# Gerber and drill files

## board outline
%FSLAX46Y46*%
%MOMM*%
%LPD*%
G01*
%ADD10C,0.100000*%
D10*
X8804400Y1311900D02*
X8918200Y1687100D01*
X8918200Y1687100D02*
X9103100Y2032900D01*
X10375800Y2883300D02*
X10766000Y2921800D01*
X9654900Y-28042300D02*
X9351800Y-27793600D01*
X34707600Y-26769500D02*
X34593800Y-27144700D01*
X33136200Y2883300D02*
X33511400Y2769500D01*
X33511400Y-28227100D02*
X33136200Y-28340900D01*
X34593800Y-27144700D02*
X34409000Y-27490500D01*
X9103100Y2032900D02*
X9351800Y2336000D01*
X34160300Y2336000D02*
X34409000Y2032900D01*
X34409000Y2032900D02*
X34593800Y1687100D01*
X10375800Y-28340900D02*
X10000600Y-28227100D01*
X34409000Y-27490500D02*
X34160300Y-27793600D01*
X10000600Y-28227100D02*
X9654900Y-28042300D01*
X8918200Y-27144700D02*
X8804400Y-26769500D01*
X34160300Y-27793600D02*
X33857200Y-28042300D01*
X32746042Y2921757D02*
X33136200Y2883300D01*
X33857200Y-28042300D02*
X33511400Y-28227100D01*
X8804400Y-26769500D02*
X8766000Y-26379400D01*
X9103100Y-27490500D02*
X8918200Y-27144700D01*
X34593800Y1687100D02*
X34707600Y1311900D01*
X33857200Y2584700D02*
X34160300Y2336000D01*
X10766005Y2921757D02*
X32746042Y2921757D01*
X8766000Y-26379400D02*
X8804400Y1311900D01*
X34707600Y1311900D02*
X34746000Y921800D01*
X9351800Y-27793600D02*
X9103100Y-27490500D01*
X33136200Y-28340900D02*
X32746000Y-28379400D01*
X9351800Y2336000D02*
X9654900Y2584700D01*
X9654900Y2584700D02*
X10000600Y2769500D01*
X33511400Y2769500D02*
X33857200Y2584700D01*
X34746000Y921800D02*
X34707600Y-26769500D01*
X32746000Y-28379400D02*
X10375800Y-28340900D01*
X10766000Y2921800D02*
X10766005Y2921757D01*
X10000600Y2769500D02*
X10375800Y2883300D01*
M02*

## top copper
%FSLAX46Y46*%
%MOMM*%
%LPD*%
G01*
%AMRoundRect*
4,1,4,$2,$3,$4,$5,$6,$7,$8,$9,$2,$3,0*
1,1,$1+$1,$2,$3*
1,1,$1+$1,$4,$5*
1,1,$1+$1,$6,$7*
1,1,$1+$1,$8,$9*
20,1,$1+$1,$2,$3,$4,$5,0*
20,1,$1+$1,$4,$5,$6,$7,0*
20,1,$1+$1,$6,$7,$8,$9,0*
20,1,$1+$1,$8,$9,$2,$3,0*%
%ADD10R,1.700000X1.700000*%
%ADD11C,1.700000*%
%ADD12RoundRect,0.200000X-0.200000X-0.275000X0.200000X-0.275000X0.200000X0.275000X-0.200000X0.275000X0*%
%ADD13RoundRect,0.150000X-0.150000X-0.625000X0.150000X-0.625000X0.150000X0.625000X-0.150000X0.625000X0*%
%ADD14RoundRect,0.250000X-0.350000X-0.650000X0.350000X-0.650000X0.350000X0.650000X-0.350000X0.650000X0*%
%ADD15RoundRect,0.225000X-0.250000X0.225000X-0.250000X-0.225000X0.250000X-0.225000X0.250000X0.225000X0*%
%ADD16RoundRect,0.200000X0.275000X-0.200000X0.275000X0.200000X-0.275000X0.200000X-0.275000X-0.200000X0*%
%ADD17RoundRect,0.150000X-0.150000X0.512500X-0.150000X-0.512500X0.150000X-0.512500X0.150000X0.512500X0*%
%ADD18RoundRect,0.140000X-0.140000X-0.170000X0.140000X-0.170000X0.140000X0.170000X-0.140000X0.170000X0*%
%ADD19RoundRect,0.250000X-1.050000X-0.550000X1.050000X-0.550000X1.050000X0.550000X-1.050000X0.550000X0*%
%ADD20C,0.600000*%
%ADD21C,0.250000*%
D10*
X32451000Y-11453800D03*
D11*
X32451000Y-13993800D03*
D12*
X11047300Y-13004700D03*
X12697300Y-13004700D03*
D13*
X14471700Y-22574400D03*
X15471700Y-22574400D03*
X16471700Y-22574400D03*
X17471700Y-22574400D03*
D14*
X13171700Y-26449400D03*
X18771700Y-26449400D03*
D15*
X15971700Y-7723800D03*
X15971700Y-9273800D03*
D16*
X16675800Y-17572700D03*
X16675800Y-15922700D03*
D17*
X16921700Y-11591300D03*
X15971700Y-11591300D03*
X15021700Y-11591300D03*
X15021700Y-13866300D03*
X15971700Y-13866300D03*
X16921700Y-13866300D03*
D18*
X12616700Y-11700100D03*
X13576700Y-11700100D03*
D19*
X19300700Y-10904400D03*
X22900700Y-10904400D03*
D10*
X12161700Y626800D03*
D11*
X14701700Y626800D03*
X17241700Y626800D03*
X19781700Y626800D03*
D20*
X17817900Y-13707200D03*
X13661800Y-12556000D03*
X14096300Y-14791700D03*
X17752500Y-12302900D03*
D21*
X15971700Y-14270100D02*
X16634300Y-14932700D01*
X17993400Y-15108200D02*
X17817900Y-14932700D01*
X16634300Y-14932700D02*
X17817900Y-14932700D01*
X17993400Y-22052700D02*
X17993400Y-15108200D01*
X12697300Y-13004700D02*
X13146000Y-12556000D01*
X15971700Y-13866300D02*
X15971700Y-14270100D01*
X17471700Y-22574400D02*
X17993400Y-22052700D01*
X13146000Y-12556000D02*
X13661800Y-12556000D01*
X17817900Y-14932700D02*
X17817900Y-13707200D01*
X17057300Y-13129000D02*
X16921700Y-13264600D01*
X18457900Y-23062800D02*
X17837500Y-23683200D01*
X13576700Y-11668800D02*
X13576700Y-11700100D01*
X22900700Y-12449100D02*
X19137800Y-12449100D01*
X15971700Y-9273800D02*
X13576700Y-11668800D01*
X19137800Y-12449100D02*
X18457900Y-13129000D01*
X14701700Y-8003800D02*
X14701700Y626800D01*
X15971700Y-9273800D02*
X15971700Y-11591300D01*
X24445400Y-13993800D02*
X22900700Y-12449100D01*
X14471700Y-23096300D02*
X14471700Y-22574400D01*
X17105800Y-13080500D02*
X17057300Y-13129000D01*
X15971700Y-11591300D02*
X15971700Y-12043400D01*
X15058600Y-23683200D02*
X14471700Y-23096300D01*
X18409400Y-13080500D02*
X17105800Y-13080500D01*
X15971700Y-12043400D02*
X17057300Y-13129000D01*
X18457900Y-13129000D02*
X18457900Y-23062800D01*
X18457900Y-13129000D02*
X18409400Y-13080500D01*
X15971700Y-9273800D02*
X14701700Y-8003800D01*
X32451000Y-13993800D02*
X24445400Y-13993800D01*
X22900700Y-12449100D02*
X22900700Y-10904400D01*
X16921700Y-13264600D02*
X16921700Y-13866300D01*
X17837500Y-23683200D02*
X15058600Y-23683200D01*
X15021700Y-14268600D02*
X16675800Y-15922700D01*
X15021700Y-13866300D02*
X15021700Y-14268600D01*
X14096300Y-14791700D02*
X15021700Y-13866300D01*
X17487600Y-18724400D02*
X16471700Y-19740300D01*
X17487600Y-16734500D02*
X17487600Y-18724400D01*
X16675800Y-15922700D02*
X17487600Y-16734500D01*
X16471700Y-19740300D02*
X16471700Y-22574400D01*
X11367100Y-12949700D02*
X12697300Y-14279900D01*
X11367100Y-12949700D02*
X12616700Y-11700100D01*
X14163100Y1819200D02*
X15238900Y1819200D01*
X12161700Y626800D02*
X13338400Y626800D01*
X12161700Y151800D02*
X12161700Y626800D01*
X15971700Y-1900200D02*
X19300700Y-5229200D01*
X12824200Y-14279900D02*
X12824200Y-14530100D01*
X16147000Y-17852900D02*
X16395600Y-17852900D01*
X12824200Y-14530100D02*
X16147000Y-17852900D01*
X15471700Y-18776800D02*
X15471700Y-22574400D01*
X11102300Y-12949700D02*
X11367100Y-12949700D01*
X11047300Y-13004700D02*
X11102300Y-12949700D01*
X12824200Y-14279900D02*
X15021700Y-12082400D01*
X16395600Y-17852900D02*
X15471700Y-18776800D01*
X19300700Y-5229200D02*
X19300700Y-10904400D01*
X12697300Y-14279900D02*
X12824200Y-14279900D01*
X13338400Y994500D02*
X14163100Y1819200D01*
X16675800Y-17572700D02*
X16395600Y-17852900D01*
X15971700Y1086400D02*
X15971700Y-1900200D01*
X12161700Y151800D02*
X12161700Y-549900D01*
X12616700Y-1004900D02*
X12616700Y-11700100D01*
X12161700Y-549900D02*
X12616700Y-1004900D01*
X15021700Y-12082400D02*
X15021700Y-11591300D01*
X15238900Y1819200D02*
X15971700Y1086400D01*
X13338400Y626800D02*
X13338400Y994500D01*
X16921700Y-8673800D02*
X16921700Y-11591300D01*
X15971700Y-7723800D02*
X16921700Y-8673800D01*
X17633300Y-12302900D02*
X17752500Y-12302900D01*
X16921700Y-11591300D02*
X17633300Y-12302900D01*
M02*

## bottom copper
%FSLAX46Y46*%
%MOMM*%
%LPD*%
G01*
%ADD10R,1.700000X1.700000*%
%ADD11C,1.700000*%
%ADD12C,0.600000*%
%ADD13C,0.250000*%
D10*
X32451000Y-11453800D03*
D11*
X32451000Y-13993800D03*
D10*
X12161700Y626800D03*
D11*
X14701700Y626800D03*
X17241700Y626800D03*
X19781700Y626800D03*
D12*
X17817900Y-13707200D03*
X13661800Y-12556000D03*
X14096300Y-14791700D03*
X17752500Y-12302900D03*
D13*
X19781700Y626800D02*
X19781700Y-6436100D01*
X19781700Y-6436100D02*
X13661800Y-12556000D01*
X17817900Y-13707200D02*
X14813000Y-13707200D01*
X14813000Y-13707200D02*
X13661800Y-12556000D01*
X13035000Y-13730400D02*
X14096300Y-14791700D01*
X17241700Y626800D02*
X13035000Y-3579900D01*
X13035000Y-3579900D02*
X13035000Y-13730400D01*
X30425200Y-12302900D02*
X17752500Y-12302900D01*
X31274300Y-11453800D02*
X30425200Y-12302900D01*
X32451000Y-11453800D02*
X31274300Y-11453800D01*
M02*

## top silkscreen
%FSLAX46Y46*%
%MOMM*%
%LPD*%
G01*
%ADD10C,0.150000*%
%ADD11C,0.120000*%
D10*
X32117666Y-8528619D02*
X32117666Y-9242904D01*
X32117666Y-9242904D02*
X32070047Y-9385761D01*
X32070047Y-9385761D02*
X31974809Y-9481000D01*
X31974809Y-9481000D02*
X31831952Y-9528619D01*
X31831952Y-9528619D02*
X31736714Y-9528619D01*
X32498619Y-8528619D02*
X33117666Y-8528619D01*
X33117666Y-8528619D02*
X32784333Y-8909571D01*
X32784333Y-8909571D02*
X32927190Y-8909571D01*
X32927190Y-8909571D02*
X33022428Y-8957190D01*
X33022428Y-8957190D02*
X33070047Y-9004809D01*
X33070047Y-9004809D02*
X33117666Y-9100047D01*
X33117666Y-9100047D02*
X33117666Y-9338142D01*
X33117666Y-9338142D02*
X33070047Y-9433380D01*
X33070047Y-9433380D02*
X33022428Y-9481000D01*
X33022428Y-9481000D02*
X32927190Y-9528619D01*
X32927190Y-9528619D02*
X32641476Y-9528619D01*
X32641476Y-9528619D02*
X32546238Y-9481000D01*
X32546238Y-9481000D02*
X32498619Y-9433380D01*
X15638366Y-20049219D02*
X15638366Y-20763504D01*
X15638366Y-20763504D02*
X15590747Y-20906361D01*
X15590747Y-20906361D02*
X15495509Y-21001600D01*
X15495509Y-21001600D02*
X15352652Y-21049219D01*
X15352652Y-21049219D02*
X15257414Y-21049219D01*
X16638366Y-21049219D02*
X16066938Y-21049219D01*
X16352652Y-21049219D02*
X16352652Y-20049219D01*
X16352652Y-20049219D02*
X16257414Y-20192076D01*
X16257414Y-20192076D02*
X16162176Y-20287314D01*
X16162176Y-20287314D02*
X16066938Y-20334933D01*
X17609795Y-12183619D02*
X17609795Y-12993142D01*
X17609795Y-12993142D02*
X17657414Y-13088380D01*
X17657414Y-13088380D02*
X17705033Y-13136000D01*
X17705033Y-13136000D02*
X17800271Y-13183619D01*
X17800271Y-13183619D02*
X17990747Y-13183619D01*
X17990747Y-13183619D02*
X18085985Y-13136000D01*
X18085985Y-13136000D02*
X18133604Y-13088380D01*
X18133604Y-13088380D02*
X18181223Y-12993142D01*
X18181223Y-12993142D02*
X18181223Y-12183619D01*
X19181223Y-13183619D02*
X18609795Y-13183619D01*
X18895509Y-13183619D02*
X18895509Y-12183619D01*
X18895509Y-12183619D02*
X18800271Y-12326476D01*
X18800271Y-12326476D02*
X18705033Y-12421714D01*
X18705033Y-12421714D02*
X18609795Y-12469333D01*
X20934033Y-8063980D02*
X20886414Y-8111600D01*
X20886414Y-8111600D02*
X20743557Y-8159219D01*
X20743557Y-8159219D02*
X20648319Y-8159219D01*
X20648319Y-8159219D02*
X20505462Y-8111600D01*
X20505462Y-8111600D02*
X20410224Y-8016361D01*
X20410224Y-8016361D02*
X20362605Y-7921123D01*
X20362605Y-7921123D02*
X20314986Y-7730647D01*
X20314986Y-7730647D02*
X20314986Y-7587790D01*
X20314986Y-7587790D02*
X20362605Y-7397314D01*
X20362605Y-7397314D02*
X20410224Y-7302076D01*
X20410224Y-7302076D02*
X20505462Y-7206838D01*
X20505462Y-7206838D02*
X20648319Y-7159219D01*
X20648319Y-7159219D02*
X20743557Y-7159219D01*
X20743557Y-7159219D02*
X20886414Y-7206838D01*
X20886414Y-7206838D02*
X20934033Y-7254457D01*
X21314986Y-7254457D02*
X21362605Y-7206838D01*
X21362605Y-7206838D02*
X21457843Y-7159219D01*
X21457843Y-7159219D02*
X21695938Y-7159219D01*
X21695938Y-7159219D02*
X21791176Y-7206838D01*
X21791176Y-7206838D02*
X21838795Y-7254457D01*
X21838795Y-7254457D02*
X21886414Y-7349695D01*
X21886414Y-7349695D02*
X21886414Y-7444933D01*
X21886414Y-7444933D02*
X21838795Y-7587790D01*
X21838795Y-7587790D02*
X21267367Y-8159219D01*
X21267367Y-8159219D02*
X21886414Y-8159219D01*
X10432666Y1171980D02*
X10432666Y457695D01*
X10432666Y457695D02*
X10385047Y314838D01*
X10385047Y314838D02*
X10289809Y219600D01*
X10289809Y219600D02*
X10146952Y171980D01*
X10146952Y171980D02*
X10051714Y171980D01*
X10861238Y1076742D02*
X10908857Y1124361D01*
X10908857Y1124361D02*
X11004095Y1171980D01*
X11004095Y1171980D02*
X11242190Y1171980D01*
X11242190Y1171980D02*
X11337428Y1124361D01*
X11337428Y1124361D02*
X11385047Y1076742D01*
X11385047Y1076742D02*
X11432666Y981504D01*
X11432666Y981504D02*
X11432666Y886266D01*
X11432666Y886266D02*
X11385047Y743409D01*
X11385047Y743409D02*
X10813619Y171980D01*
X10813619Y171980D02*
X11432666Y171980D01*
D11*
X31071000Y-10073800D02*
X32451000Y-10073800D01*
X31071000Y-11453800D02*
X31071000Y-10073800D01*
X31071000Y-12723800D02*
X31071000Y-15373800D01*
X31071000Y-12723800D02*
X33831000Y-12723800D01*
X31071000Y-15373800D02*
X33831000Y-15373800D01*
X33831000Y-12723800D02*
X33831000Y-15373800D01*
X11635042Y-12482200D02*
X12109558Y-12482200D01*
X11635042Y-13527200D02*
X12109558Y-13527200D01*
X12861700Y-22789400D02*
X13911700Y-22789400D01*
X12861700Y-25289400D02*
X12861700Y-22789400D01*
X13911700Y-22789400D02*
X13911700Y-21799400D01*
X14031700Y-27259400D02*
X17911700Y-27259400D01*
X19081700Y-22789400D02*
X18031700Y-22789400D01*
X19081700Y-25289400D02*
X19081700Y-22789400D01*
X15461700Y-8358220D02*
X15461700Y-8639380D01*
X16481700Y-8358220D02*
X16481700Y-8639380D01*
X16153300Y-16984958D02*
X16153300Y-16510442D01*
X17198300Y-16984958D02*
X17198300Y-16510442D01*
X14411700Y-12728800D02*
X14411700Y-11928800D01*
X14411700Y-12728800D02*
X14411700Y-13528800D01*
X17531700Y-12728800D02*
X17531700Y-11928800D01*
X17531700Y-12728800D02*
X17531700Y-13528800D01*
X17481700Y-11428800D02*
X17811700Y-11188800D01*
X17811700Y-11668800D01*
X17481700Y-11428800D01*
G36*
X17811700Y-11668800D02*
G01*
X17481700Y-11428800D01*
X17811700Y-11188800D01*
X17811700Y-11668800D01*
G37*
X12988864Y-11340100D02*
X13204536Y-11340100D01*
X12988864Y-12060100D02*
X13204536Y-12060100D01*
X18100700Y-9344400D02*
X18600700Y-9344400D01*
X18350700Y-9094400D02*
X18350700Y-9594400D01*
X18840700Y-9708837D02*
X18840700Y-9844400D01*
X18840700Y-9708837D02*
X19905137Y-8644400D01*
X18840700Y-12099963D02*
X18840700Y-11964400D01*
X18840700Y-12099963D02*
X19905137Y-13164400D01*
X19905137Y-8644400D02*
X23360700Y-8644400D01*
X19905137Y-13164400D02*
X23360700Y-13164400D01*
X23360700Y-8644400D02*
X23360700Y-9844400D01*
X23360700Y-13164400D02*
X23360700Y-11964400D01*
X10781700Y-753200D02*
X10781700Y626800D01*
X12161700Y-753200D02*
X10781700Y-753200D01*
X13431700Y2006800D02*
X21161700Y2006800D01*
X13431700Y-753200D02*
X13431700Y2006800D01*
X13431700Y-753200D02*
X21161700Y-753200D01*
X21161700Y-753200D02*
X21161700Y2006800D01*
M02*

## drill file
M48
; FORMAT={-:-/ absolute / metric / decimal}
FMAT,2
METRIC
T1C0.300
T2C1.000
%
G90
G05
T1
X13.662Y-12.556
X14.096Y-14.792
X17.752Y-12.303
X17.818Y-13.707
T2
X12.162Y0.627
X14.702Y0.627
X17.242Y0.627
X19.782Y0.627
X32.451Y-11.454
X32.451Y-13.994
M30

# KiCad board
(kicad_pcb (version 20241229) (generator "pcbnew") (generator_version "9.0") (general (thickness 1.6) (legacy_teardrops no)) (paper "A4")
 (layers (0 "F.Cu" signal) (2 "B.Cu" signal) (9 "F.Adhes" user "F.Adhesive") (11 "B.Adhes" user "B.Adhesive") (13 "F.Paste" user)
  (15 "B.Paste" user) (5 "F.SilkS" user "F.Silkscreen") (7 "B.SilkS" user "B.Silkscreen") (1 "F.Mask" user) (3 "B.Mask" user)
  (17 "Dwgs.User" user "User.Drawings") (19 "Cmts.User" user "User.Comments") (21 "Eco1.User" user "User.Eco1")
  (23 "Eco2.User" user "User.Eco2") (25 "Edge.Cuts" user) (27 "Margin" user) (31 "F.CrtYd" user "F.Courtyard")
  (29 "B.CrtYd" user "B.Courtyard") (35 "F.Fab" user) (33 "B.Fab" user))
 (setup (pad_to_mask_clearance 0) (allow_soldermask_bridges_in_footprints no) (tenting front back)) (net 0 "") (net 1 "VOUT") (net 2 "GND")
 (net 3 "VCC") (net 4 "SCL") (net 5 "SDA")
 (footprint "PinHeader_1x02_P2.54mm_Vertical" (layer "F.Cu") (at 32.451 11.4538)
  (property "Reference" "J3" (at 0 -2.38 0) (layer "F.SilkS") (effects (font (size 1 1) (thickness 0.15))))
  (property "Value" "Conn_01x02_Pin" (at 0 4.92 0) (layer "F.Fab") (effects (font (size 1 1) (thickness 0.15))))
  (fp_line (start -1.38 -1.38) (end 0 -1.38) (stroke (width 0.12) (type solid)) (layer "F.SilkS"))
  (fp_line (start -1.38 0) (end -1.38 -1.38) (stroke (width 0.12) (type solid)) (layer "F.SilkS"))
  (fp_line (start -1.38 1.27) (end -1.38 3.92) (stroke (width 0.12) (type solid)) (layer "F.SilkS"))
  (fp_line (start -1.38 1.27) (end 1.38 1.27) (stroke (width 0.12) (type solid)) (layer "F.SilkS"))
  (fp_line (start -1.38 3.92) (end 1.38 3.92) (stroke (width 0.12) (type solid)) (layer "F.SilkS"))
  (fp_line (start 1.38 1.27) (end 1.38 3.92) (stroke (width 0.12) (type solid)) (layer "F.SilkS"))
  (pad "1" thru_hole rect (at 0 0) (size 1.7 1.7) (drill 1) (layers "*.Cu" "*.Mask") (remove_unused_layers no) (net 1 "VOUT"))
  (pad "2" thru_hole circle (at 0 2.54) (size 1.7 1.7) (drill 1) (layers "*.Cu" "*.Mask") (remove_unused_layers no) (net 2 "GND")))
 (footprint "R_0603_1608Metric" (layer "F.Cu") (at 11.8723 13.0047)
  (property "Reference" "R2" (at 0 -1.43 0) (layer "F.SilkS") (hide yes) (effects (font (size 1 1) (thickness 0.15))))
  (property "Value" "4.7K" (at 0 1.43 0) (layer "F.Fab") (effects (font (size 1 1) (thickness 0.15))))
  (fp_line (start -0.237258 -0.5225) (end 0.237258 -0.5225) (stroke (width 0.12) (type solid)) (layer "F.SilkS"))
  (fp_line (start -0.237258 0.5225) (end 0.237258 0.5225) (stroke (width 0.12) (type solid)) (layer "F.SilkS"))
  (pad "1" smd roundrect (at -0.825 0) (size 0.8 0.95) (layers "F.Cu" "F.Mask" "F.Paste") (roundrect_rratio 0.25) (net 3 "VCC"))
  (pad "2" smd roundrect (at 0.825 0) (size 0.8 0.95) (layers "F.Cu" "F.Mask" "F.Paste") (roundrect_rratio 0.25) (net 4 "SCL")))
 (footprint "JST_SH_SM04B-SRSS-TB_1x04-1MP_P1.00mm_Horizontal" (layer "F.Cu") (at 15.9717 24.5744)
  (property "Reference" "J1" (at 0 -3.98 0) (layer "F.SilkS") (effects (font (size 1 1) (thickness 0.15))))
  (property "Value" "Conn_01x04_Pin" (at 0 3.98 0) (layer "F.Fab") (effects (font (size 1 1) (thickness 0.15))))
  (fp_line (start -3.11 -1.785) (end -2.06 -1.785) (stroke (width 0.12) (type solid)) (layer "F.SilkS"))
  (fp_line (start -3.11 0.715) (end -3.11 -1.785) (stroke (width 0.12) (type solid)) (layer "F.SilkS"))
  (fp_line (start -2.06 -1.785) (end -2.06 -2.775) (stroke (width 0.12) (type solid)) (layer "F.SilkS"))
  (fp_line (start -1.94 2.685) (end 1.94 2.685) (stroke (width 0.12) (type solid)) (layer "F.SilkS"))
  (fp_line (start 3.11 -1.785) (end 2.06 -1.785) (stroke (width 0.12) (type solid)) (layer "F.SilkS"))
  (fp_line (start 3.11 0.715) (end 3.11 -1.785) (stroke (width 0.12) (type solid)) (layer "F.SilkS"))
  (pad "1" smd roundrect (at -1.5 -2) (size 0.6 1.55) (layers "F.Cu" "F.Mask" "F.Paste") (roundrect_rratio 0.25) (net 2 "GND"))
  (pad "2" smd roundrect (at -0.5 -2) (size 0.6 1.55) (layers "F.Cu" "F.Mask" "F.Paste") (roundrect_rratio 0.25) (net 3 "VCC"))
  (pad "3" smd roundrect (at 0.5 -2) (size 0.6 1.55) (layers "F.Cu" "F.Mask" "F.Paste") (roundrect_rratio 0.25) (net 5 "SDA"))
  (pad "4" smd roundrect (at 1.5 -2) (size 0.6 1.55) (layers "F.Cu" "F.Mask" "F.Paste") (roundrect_rratio 0.25) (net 4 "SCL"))
  (pad "MP" smd roundrect (at -2.8 1.875) (size 1.2 1.8) (layers "F.Cu" "F.Mask" "F.Paste") (roundrect_rratio 0.208333))
  (pad "MP" smd roundrect (at 2.8 1.875) (size 1.2 1.8) (layers "F.Cu" "F.Mask" "F.Paste") (roundrect_rratio 0.208333)))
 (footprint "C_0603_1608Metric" (layer "F.Cu") (at 15.9717 8.4988 -90)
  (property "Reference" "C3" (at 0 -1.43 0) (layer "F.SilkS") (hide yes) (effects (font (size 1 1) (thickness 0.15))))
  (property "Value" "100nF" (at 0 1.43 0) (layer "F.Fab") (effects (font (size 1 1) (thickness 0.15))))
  (fp_line (start -0.14058 0.51) (end 0.14058 0.51) (stroke (width 0.12) (type solid)) (layer "F.SilkS"))
  (fp_line (start -0.14058 -0.51) (end 0.14058 -0.51) (stroke (width 0.12) (type solid)) (layer "F.SilkS"))
  (pad "1" smd roundrect (at -0.775 0 270) (size 0.9 0.95) (layers "F.Cu" "F.Mask" "F.Paste") (roundrect_rratio 0.25) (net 1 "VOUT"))
  (pad "2" smd roundrect (at 0.775 0 270) (size 0.9 0.95) (layers "F.Cu" "F.Mask" "F.Paste") (roundrect_rratio 0.25) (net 2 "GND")))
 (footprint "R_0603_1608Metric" (layer "F.Cu") (at 16.6758 16.7477 90)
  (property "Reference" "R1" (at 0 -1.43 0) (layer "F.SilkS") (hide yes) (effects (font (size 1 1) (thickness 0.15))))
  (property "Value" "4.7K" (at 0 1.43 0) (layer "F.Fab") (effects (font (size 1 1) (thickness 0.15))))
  (fp_line (start -0.237258 -0.5225) (end 0.237258 -0.5225) (stroke (width 0.12) (type solid)) (layer "F.SilkS"))
  (fp_line (start -0.237258 0.5225) (end 0.237258 0.5225) (stroke (width 0.12) (type solid)) (layer "F.SilkS"))
  (pad "1" smd roundrect (at -0.825 0 90) (size 0.8 0.95) (layers "F.Cu" "F.Mask" "F.Paste") (roundrect_rratio 0.25) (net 3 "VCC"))
  (pad "2" smd roundrect (at 0.825 0 90) (size 0.8 0.95) (layers "F.Cu" "F.Mask" "F.Paste") (roundrect_rratio 0.25) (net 5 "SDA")))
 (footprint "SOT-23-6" (layer "F.Cu") (at 15.9717 12.7288 -90)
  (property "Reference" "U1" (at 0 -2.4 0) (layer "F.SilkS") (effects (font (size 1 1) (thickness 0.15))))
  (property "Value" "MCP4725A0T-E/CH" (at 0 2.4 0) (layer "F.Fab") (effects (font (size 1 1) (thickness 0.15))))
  (fp_line (start 0 1.56) (end -0.8 1.56) (stroke (width 0.12) (type solid)) (layer "F.SilkS"))
  (fp_line (start 0 1.56) (end 0.8 1.56) (stroke (width 0.12) (type solid)) (layer "F.SilkS"))
  (fp_line (start 0 -1.56) (end -0.8 -1.56) (stroke (width 0.12) (type solid)) (layer "F.SilkS"))
  (fp_line (start 0 -1.56) (end 0.8 -1.56) (stroke (width 0.12) (type solid)) (layer "F.SilkS"))
  (fp_poly (pts (xy -1.3 -1.51) (xy -1.54 -1.84) (xy -1.06 -1.84)) (stroke (width 0.12) (type solid)) (fill yes) (layer "F.SilkS"))
  (pad "1" smd roundrect (at -1.1375 -0.95 270) (size 1.325 0.6) (layers "F.Cu" "F.Mask" "F.Paste") (roundrect_rratio 0.25) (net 1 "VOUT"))
  (pad "2" smd roundrect (at -1.1375 0 270) (size 1.325 0.6) (layers "F.Cu" "F.Mask" "F.Paste") (roundrect_rratio 0.25) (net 2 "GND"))
  (pad "3" smd roundrect (at -1.1375 0.95 270) (size 1.325 0.6) (layers "F.Cu" "F.Mask" "F.Paste") (roundrect_rratio 0.25) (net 3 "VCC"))
  (pad "4" smd roundrect (at 1.1375 0.95 270) (size 1.325 0.6) (layers "F.Cu" "F.Mask" "F.Paste") (roundrect_rratio 0.25) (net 5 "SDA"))
  (pad "5" smd roundrect (at 1.1375 0 270) (size 1.325 0.6) (layers "F.Cu" "F.Mask" "F.Paste") (roundrect_rratio 0.25) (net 4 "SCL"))
  (pad "6" smd roundrect (at 1.1375 -0.95 270) (size 1.325 0.6) (layers "F.Cu" "F.Mask" "F.Paste") (roundrect_rratio 0.25) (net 2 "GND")))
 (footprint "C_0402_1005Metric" (layer "F.Cu") (at 13.0967 11.7001)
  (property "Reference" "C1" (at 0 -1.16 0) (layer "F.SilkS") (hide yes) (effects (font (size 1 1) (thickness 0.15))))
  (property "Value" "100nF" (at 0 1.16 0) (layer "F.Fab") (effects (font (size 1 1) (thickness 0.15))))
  (fp_line (start -0.107836 -0.36) (end 0.107836 -0.36) (stroke (width 0.12) (type solid)) (layer "F.SilkS"))
  (fp_line (start -0.107836 0.36) (end 0.107836 0.36) (stroke (width 0.12) (type solid)) (layer "F.SilkS"))
  (pad "1" smd roundrect (at -0.48 0) (size 0.56 0.62) (layers "F.Cu" "F.Mask" "F.Paste") (roundrect_rratio 0.25) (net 3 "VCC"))
  (pad "2" smd roundrect (at 0.48 0) (size 0.56 0.62) (layers "F.Cu" "F.Mask" "F.Paste") (roundrect_rratio 0.25) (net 2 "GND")))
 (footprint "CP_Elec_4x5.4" (layer "F.Cu") (at 21.1007 10.9044)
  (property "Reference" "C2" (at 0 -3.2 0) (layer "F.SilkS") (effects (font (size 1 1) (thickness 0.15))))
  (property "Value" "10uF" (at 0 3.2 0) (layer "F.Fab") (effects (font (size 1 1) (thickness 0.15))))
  (fp_line (start -3 -1.56) (end -2.5 -1.56) (stroke (width 0.12) (type solid)) (layer "F.SilkS"))
  (fp_line (start -2.75 -1.81) (end -2.75 -1.31) (stroke (width 0.12) (type solid)) (layer "F.SilkS"))
  (fp_line (start -2.26 -1.195563) (end -2.26 -1.06) (stroke (width 0.12) (type solid)) (layer "F.SilkS"))
  (fp_line (start -2.26 -1.195563) (end -1.195563 -2.26) (stroke (width 0.12) (type solid)) (layer "F.SilkS"))
  (fp_line (start -2.26 1.195563) (end -2.26 1.06) (stroke (width 0.12) (type solid)) (layer "F.SilkS"))
  (fp_line (start -2.26 1.195563) (end -1.195563 2.26) (stroke (width 0.12) (type solid)) (layer "F.SilkS"))
  (fp_line (start -1.195563 -2.26) (end 2.26 -2.26) (stroke (width 0.12) (type solid)) (layer "F.SilkS"))
  (fp_line (start -1.195563 2.26) (end 2.26 2.26) (stroke (width 0.12) (type solid)) (layer "F.SilkS"))
  (fp_line (start 2.26 -2.26) (end 2.26 -1.06) (stroke (width 0.12) (type solid)) (layer "F.SilkS"))
  (fp_line (start 2.26 2.26) (end 2.26 1.06) (stroke (width 0.12) (type solid)) (layer "F.SilkS"))
  (pad "1" smd roundrect (at -1.8 0) (size 2.6 1.6) (layers "F.Cu" "F.Mask" "F.Paste") (roundrect_rratio 0.15625) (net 3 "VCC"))
  (pad "2" smd roundrect (at 1.8 0) (size 2.6 1.6) (layers "F.Cu" "F.Mask" "F.Paste") (roundrect_rratio 0.15625) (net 2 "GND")))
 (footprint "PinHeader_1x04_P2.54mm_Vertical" (layer "F.Cu") (at 12.1617 -0.6268 90)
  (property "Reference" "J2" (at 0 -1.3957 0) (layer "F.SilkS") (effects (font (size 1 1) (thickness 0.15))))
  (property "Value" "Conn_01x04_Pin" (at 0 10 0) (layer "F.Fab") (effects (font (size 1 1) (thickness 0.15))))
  (fp_line (start -1.38 -1.38) (end 0 -1.38) (stroke (width 0.12) (type solid)) (layer "F.SilkS"))
  (fp_line (start -1.38 0) (end -1.38 -1.38) (stroke (width 0.12) (type solid)) (layer "F.SilkS"))
  (fp_line (start 1.38 1.27) (end 1.38 9) (stroke (width 0.12) (type solid)) (layer "F.SilkS"))
  (fp_line (start -1.38 1.27) (end 1.38 1.27) (stroke (width 0.12) (type solid)) (layer "F.SilkS"))
  (fp_line (start -1.38 1.27) (end -1.38 9) (stroke (width 0.12) (type solid)) (layer "F.SilkS"))
  (fp_line (start -1.38 9) (end 1.38 9) (stroke (width 0.12) (type solid)) (layer "F.SilkS"))
  (pad "1" thru_hole rect (at 0 0 90) (size 1.7 1.7) (drill 1) (layers "*.Cu" "*.Mask") (remove_unused_layers no) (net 3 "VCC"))
  (pad "2" thru_hole circle (at 0 2.54 90) (size 1.7 1.7) (drill 1) (layers "*.Cu" "*.Mask") (remove_unused_layers no) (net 2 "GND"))
  (pad "3" thru_hole circle (at 0 5.08 90) (size 1.7 1.7) (drill 1) (layers "*.Cu" "*.Mask") (remove_unused_layers no) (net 5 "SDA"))
  (pad "4" thru_hole circle (at 0 7.62 90) (size 1.7 1.7) (drill 1) (layers "*.Cu" "*.Mask") (remove_unused_layers no) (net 4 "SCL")))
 (gr_line (start 8.8044 -1.3119) (end 8.9182 -1.6871) (stroke (width 0.1) (type solid)) (layer "Edge.Cuts"))
 (gr_line (start 8.9182 -1.6871) (end 9.1031 -2.0329) (stroke (width 0.1) (type solid)) (layer "Edge.Cuts"))
 (gr_line (start 10.3758 -2.8833) (end 10.766 -2.9218) (stroke (width 0.1) (type solid)) (layer "Edge.Cuts"))
 (gr_line (start 9.6549 28.0423) (end 9.3518 27.7936) (stroke (width 0.1) (type solid)) (layer "Edge.Cuts"))
 (gr_line (start 34.7076 26.7695) (end 34.5938 27.1447) (stroke (width 0.1) (type solid)) (layer "Edge.Cuts"))
 (gr_line (start 33.1362 -2.8833) (end 33.5114 -2.7695) (stroke (width 0.1) (type solid)) (layer "Edge.Cuts"))
 (gr_line (start 33.5114 28.2271) (end 33.1362 28.3409) (stroke (width 0.1) (type solid)) (layer "Edge.Cuts"))
 (gr_line (start 34.5938 27.1447) (end 34.409 27.4905) (stroke (width 0.1) (type solid)) (layer "Edge.Cuts"))
 (gr_line (start 9.1031 -2.0329) (end 9.3518 -2.336) (stroke (width 0.1) (type solid)) (layer "Edge.Cuts"))
 (gr_line (start 34.1603 -2.336) (end 34.409 -2.0329) (stroke (width 0.1) (type solid)) (layer "Edge.Cuts"))
 (gr_line (start 34.409 -2.0329) (end 34.5938 -1.6871) (stroke (width 0.1) (type solid)) (layer "Edge.Cuts"))
 (gr_line (start 10.3758 28.3409) (end 10.0006 28.2271) (stroke (width 0.1) (type solid)) (layer "Edge.Cuts"))
 (gr_line (start 34.409 27.4905) (end 34.1603 27.7936) (stroke (width 0.1) (type solid)) (layer "Edge.Cuts"))
 (gr_line (start 10.0006 28.2271) (end 9.6549 28.0423) (stroke (width 0.1) (type solid)) (layer "Edge.Cuts"))
 (gr_line (start 8.9182 27.1447) (end 8.8044 26.7695) (stroke (width 0.1) (type solid)) (layer "Edge.Cuts"))
 (gr_line (start 34.1603 27.7936) (end 33.8572 28.0423) (stroke (width 0.1) (type solid)) (layer "Edge.Cuts"))
 (gr_line (start 32.746042 -2.921757) (end 33.1362 -2.8833) (stroke (width 0.1) (type solid)) (layer "Edge.Cuts"))
 (gr_line (start 33.8572 28.0423) (end 33.5114 28.2271) (stroke (width 0.1) (type solid)) (layer "Edge.Cuts"))
 (gr_line (start 8.8044 26.7695) (end 8.766 26.3794) (stroke (width 0.1) (type solid)) (layer "Edge.Cuts"))
 (gr_line (start 9.1031 27.4905) (end 8.9182 27.1447) (stroke (width 0.1) (type solid)) (layer "Edge.Cuts"))
 (gr_line (start 34.5938 -1.6871) (end 34.7076 -1.3119) (stroke (width 0.1) (type solid)) (layer "Edge.Cuts"))
 (gr_line (start 33.8572 -2.5847) (end 34.1603 -2.336) (stroke (width 0.1) (type solid)) (layer "Edge.Cuts"))
 (gr_line (start 10.766005 -2.921757) (end 32.746042 -2.921757) (stroke (width 0.1) (type solid)) (layer "Edge.Cuts"))
 (gr_line (start 8.766 26.3794) (end 8.8044 -1.3119) (stroke (width 0.1) (type solid)) (layer "Edge.Cuts"))
 (gr_line (start 34.7076 -1.3119) (end 34.746 -0.9218) (stroke (width 0.1) (type solid)) (layer "Edge.Cuts"))
 (gr_line (start 9.3518 27.7936) (end 9.1031 27.4905) (stroke (width 0.1) (type solid)) (layer "Edge.Cuts"))
 (gr_line (start 33.1362 28.3409) (end 32.746 28.3794) (stroke (width 0.1) (type solid)) (layer "Edge.Cuts"))
 (gr_line (start 9.3518 -2.336) (end 9.6549 -2.5847) (stroke (width 0.1) (type solid)) (layer "Edge.Cuts"))
 (gr_line (start 9.6549 -2.5847) (end 10.0006 -2.7695) (stroke (width 0.1) (type solid)) (layer "Edge.Cuts"))
 (gr_line (start 33.5114 -2.7695) (end 33.8572 -2.5847) (stroke (width 0.1) (type solid)) (layer "Edge.Cuts"))
 (gr_line (start 34.746 -0.9218) (end 34.7076 26.7695) (stroke (width 0.1) (type solid)) (layer "Edge.Cuts"))
 (gr_line (start 32.746 28.3794) (end 10.3758 28.3409) (stroke (width 0.1) (type solid)) (layer "Edge.Cuts"))
 (gr_line (start 10.766 -2.9218) (end 10.766005 -2.921757) (stroke (width 0.1) (type solid)) (layer "Edge.Cuts"))
 (gr_line (start 10.0006 -2.7695) (end 10.3758 -2.8833) (stroke (width 0.1) (type solid)) (layer "Edge.Cuts"))
 (segment (start 15.9717 14.2701) (end 16.6343 14.9327) (width 0.25) (layer "F.Cu") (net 4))
 (segment (start 17.9934 15.1082) (end 17.8179 14.9327) (width 0.25) (layer "F.Cu") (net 4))
 (segment (start 16.6343 14.9327) (end 17.8179 14.9327) (width 0.25) (layer "F.Cu") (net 4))
 (segment (start 17.9934 22.0527) (end 17.9934 15.1082) (width 0.25) (layer "F.Cu") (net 4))
 (segment (start 12.6973 13.0047) (end 13.146 12.556) (width 0.25) (layer "F.Cu") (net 4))
 (segment (start 15.9717 13.8663) (end 15.9717 14.2701) (width 0.25) (layer "F.Cu") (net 4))
 (segment (start 17.4717 22.5744) (end 17.9934 22.0527) (width 0.25) (layer "F.Cu") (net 4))
 (segment (start 13.146 12.556) (end 13.6618 12.556) (width 0.25) (layer "F.Cu") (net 4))
 (segment (start 17.8179 14.9327) (end 17.8179 13.7072) (width 0.25) (layer "F.Cu") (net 4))
 (via (at 17.8179 13.7072) (size 0.6) (drill 0.3) (layers "F.Cu" "B.Cu") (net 4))
 (via (at 13.6618 12.556) (size 0.6) (drill 0.3) (layers "F.Cu" "B.Cu") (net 4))
 (segment (start 19.7817 -0.6268) (end 19.7817 6.4361) (width 0.25) (layer "B.Cu") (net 4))
 (segment (start 19.7817 6.4361) (end 13.6618 12.556) (width 0.25) (layer "B.Cu") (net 4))
 (segment (start 17.8179 13.7072) (end 14.813 13.7072) (width 0.25) (layer "B.Cu") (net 4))
 (segment (start 14.813 13.7072) (end 13.6618 12.556) (width 0.25) (layer "B.Cu") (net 4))
 (segment (start 17.0573 13.129) (end 16.9217 13.2646) (width 0.25) (layer "F.Cu") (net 2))
 (segment (start 18.4579 23.0628) (end 17.8375 23.6832) (width 0.25) (layer "F.Cu") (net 2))
 (segment (start 13.5767 11.6688) (end 13.5767 11.7001) (width 0.25) (layer "F.Cu") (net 2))
 (segment (start 22.9007 12.4491) (end 19.1378 12.4491) (width 0.25) (layer "F.Cu") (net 2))
 (segment (start 15.9717 9.2738) (end 13.5767 11.6688) (width 0.25) (layer "F.Cu") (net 2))
 (segment (start 19.1378 12.4491) (end 18.4579 13.129) (width 0.25) (layer "F.Cu") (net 2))
 (segment (start 14.7017 8.0038) (end 14.7017 -0.6268) (width 0.25) (layer "F.Cu") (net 2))
 (segment (start 15.9717 9.2738) (end 15.9717 11.5913) (width 0.25) (layer "F.Cu") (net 2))
 (segment (start 24.4454 13.9938) (end 22.9007 12.4491) (width 0.25) (layer "F.Cu") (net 2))
 (segment (start 14.4717 23.0963) (end 14.4717 22.5744) (width 0.25) (layer "F.Cu") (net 2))
 (segment (start 17.1058 13.0805) (end 17.0573 13.129) (width 0.25) (layer "F.Cu") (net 2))
 (segment (start 15.9717 11.5913) (end 15.9717 12.0434) (width 0.25) (layer "F.Cu") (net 2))
 (segment (start 15.0586 23.6832) (end 14.4717 23.0963) (width 0.25) (layer "F.Cu") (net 2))
 (segment (start 18.4094 13.0805) (end 17.1058 13.0805) (width 0.25) (layer "F.Cu") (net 2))
 (segment (start 15.9717 12.0434) (end 17.0573 13.129) (width 0.25) (layer "F.Cu") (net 2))
 (segment (start 18.4579 13.129) (end 18.4579 23.0628) (width 0.25) (layer "F.Cu") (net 2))
 (segment (start 18.4579 13.129) (end 18.4094 13.0805) (width 0.25) (layer "F.Cu") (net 2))
 (segment (start 15.9717 9.2738) (end 14.7017 8.0038) (width 0.25) (layer "F.Cu") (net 2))
 (segment (start 32.451 13.9938) (end 24.4454 13.9938) (width 0.25) (layer "F.Cu") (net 2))
 (segment (start 22.9007 12.4491) (end 22.9007 10.9044) (width 0.25) (layer "F.Cu") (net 2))
 (segment (start 16.9217 13.2646) (end 16.9217 13.8663) (width 0.25) (layer "F.Cu") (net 2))
 (segment (start 17.8375 23.6832) (end 15.0586 23.6832) (width 0.25) (layer "F.Cu") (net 2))
 (segment (start 15.0217 14.2686) (end 16.6758 15.9227) (width 0.25) (layer "F.Cu") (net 5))
 (segment (start 15.0217 13.8663) (end 15.0217 14.2686) (width 0.25) (layer "F.Cu") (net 5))
 (segment (start 14.0963 14.7917) (end 15.0217 13.8663) (width 0.25) (layer "F.Cu") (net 5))
 (segment (start 17.4876 18.7244) (end 16.4717 19.7403) (width 0.25) (layer "F.Cu") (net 5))
 (segment (start 17.4876 16.7345) (end 17.4876 18.7244) (width 0.25) (layer "F.Cu") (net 5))
 (segment (start 16.6758 15.9227) (end 17.4876 16.7345) (width 0.25) (layer "F.Cu") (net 5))
 (segment (start 16.4717 19.7403) (end 16.4717 22.5744) (width 0.25) (layer "F.Cu") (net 5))
 (via (at 14.0963 14.7917) (size 0.6) (drill 0.3) (layers "F.Cu" "B.Cu") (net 5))
 (segment (start 13.035 13.7304) (end 14.0963 14.7917) (width 0.25) (layer "B.Cu") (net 5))
 (segment (start 17.2417 -0.6268) (end 13.035 3.5799) (width 0.25) (layer "B.Cu") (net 5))
 (segment (start 13.035 3.5799) (end 13.035 13.7304) (width 0.25) (layer "B.Cu") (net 5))
 (segment (start 11.3671 12.9497) (end 12.6973 14.2799) (width 0.25) (layer "F.Cu") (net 3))
 (segment (start 11.3671 12.9497) (end 12.6167 11.7001) (width 0.25) (layer "F.Cu") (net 3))
 (segment (start 14.1631 -1.8192) (end 15.2389 -1.8192) (width 0.25) (layer "F.Cu") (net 3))
 (segment (start 12.1617 -0.6268) (end 13.3384 -0.6268) (width 0.25) (layer "F.Cu") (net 3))
 (segment (start 12.1617 -0.1518) (end 12.1617 -0.6268) (width 0.25) (layer "F.Cu") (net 3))
 (segment (start 15.9717 1.9002) (end 19.3007 5.2292) (width 0.25) (layer "F.Cu") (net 3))
 (segment (start 12.8242 14.2799) (end 12.8242 14.5301) (width 0.25) (layer "F.Cu") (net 3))
 (segment (start 16.147 17.8529) (end 16.3956 17.8529) (width 0.25) (layer "F.Cu") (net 3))
 (segment (start 12.8242 14.5301) (end 16.147 17.8529) (width 0.25) (layer "F.Cu") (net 3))
 (segment (start 15.4717 18.7768) (end 15.4717 22.5744) (width 0.25) (layer "F.Cu") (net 3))
 (segment (start 11.1023 12.9497) (end 11.3671 12.9497) (width 0.25) (layer "F.Cu") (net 3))
 (segment (start 11.0473 13.0047) (end 11.1023 12.9497) (width 0.25) (layer "F.Cu") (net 3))
 (segment (start 12.8242 14.2799) (end 15.0217 12.0824) (width 0.25) (layer "F.Cu") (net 3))
 (segment (start 16.3956 17.8529) (end 15.4717 18.7768) (width 0.25) (layer "F.Cu") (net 3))
 (segment (start 19.3007 5.2292) (end 19.3007 10.9044) (width 0.25) (layer "F.Cu") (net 3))
 (segment (start 12.6973 14.2799) (end 12.8242 14.2799) (width 0.25) (layer "F.Cu") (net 3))
 (segment (start 13.3384 -0.9945) (end 14.1631 -1.8192) (width 0.25) (layer "F.Cu") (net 3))
 (segment (start 16.6758 17.5727) (end 16.3956 17.8529) (width 0.25) (layer "F.Cu") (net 3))
 (segment (start 15.9717 -1.0864) (end 15.9717 1.9002) (width 0.25) (layer "F.Cu") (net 3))
 (segment (start 12.1617 -0.1518) (end 12.1617 0.5499) (width 0.25) (layer "F.Cu") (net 3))
 (segment (start 12.6167 1.0049) (end 12.6167 11.7001) (width 0.25) (layer "F.Cu") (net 3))
 (segment (start 12.1617 0.5499) (end 12.6167 1.0049) (width 0.25) (layer "F.Cu") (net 3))
 (segment (start 15.0217 12.0824) (end 15.0217 11.5913) (width 0.25) (layer "F.Cu") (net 3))
 (segment (start 15.2389 -1.8192) (end 15.9717 -1.0864) (width 0.25) (layer "F.Cu") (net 3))
 (segment (start 13.3384 -0.6268) (end 13.3384 -0.9945) (width 0.25) (layer "F.Cu") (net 3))
 (segment (start 16.9217 8.6738) (end 16.9217 11.5913) (width 0.25) (layer "F.Cu") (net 1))
 (segment (start 15.9717 7.7238) (end 16.9217 8.6738) (width 0.25) (layer "F.Cu") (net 1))
 (segment (start 17.6333 12.3029) (end 17.7525 12.3029) (width 0.25) (layer "F.Cu") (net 1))
 (segment (start 16.9217 11.5913) (end 17.6333 12.3029) (width 0.25) (layer "F.Cu") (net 1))
 (via (at 17.7525 12.3029) (size 0.6) (drill 0.3) (layers "F.Cu" "B.Cu") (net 1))
 (segment (start 30.4252 12.3029) (end 17.7525 12.3029) (width 0.25) (layer "B.Cu") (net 1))
 (segment (start 31.2743 11.4538) (end 30.4252 12.3029) (width 0.25) (layer "B.Cu") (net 1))
 (segment (start 32.451 11.4538) (end 31.2743 11.4538) (width 0.25) (layer "B.Cu") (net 1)))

